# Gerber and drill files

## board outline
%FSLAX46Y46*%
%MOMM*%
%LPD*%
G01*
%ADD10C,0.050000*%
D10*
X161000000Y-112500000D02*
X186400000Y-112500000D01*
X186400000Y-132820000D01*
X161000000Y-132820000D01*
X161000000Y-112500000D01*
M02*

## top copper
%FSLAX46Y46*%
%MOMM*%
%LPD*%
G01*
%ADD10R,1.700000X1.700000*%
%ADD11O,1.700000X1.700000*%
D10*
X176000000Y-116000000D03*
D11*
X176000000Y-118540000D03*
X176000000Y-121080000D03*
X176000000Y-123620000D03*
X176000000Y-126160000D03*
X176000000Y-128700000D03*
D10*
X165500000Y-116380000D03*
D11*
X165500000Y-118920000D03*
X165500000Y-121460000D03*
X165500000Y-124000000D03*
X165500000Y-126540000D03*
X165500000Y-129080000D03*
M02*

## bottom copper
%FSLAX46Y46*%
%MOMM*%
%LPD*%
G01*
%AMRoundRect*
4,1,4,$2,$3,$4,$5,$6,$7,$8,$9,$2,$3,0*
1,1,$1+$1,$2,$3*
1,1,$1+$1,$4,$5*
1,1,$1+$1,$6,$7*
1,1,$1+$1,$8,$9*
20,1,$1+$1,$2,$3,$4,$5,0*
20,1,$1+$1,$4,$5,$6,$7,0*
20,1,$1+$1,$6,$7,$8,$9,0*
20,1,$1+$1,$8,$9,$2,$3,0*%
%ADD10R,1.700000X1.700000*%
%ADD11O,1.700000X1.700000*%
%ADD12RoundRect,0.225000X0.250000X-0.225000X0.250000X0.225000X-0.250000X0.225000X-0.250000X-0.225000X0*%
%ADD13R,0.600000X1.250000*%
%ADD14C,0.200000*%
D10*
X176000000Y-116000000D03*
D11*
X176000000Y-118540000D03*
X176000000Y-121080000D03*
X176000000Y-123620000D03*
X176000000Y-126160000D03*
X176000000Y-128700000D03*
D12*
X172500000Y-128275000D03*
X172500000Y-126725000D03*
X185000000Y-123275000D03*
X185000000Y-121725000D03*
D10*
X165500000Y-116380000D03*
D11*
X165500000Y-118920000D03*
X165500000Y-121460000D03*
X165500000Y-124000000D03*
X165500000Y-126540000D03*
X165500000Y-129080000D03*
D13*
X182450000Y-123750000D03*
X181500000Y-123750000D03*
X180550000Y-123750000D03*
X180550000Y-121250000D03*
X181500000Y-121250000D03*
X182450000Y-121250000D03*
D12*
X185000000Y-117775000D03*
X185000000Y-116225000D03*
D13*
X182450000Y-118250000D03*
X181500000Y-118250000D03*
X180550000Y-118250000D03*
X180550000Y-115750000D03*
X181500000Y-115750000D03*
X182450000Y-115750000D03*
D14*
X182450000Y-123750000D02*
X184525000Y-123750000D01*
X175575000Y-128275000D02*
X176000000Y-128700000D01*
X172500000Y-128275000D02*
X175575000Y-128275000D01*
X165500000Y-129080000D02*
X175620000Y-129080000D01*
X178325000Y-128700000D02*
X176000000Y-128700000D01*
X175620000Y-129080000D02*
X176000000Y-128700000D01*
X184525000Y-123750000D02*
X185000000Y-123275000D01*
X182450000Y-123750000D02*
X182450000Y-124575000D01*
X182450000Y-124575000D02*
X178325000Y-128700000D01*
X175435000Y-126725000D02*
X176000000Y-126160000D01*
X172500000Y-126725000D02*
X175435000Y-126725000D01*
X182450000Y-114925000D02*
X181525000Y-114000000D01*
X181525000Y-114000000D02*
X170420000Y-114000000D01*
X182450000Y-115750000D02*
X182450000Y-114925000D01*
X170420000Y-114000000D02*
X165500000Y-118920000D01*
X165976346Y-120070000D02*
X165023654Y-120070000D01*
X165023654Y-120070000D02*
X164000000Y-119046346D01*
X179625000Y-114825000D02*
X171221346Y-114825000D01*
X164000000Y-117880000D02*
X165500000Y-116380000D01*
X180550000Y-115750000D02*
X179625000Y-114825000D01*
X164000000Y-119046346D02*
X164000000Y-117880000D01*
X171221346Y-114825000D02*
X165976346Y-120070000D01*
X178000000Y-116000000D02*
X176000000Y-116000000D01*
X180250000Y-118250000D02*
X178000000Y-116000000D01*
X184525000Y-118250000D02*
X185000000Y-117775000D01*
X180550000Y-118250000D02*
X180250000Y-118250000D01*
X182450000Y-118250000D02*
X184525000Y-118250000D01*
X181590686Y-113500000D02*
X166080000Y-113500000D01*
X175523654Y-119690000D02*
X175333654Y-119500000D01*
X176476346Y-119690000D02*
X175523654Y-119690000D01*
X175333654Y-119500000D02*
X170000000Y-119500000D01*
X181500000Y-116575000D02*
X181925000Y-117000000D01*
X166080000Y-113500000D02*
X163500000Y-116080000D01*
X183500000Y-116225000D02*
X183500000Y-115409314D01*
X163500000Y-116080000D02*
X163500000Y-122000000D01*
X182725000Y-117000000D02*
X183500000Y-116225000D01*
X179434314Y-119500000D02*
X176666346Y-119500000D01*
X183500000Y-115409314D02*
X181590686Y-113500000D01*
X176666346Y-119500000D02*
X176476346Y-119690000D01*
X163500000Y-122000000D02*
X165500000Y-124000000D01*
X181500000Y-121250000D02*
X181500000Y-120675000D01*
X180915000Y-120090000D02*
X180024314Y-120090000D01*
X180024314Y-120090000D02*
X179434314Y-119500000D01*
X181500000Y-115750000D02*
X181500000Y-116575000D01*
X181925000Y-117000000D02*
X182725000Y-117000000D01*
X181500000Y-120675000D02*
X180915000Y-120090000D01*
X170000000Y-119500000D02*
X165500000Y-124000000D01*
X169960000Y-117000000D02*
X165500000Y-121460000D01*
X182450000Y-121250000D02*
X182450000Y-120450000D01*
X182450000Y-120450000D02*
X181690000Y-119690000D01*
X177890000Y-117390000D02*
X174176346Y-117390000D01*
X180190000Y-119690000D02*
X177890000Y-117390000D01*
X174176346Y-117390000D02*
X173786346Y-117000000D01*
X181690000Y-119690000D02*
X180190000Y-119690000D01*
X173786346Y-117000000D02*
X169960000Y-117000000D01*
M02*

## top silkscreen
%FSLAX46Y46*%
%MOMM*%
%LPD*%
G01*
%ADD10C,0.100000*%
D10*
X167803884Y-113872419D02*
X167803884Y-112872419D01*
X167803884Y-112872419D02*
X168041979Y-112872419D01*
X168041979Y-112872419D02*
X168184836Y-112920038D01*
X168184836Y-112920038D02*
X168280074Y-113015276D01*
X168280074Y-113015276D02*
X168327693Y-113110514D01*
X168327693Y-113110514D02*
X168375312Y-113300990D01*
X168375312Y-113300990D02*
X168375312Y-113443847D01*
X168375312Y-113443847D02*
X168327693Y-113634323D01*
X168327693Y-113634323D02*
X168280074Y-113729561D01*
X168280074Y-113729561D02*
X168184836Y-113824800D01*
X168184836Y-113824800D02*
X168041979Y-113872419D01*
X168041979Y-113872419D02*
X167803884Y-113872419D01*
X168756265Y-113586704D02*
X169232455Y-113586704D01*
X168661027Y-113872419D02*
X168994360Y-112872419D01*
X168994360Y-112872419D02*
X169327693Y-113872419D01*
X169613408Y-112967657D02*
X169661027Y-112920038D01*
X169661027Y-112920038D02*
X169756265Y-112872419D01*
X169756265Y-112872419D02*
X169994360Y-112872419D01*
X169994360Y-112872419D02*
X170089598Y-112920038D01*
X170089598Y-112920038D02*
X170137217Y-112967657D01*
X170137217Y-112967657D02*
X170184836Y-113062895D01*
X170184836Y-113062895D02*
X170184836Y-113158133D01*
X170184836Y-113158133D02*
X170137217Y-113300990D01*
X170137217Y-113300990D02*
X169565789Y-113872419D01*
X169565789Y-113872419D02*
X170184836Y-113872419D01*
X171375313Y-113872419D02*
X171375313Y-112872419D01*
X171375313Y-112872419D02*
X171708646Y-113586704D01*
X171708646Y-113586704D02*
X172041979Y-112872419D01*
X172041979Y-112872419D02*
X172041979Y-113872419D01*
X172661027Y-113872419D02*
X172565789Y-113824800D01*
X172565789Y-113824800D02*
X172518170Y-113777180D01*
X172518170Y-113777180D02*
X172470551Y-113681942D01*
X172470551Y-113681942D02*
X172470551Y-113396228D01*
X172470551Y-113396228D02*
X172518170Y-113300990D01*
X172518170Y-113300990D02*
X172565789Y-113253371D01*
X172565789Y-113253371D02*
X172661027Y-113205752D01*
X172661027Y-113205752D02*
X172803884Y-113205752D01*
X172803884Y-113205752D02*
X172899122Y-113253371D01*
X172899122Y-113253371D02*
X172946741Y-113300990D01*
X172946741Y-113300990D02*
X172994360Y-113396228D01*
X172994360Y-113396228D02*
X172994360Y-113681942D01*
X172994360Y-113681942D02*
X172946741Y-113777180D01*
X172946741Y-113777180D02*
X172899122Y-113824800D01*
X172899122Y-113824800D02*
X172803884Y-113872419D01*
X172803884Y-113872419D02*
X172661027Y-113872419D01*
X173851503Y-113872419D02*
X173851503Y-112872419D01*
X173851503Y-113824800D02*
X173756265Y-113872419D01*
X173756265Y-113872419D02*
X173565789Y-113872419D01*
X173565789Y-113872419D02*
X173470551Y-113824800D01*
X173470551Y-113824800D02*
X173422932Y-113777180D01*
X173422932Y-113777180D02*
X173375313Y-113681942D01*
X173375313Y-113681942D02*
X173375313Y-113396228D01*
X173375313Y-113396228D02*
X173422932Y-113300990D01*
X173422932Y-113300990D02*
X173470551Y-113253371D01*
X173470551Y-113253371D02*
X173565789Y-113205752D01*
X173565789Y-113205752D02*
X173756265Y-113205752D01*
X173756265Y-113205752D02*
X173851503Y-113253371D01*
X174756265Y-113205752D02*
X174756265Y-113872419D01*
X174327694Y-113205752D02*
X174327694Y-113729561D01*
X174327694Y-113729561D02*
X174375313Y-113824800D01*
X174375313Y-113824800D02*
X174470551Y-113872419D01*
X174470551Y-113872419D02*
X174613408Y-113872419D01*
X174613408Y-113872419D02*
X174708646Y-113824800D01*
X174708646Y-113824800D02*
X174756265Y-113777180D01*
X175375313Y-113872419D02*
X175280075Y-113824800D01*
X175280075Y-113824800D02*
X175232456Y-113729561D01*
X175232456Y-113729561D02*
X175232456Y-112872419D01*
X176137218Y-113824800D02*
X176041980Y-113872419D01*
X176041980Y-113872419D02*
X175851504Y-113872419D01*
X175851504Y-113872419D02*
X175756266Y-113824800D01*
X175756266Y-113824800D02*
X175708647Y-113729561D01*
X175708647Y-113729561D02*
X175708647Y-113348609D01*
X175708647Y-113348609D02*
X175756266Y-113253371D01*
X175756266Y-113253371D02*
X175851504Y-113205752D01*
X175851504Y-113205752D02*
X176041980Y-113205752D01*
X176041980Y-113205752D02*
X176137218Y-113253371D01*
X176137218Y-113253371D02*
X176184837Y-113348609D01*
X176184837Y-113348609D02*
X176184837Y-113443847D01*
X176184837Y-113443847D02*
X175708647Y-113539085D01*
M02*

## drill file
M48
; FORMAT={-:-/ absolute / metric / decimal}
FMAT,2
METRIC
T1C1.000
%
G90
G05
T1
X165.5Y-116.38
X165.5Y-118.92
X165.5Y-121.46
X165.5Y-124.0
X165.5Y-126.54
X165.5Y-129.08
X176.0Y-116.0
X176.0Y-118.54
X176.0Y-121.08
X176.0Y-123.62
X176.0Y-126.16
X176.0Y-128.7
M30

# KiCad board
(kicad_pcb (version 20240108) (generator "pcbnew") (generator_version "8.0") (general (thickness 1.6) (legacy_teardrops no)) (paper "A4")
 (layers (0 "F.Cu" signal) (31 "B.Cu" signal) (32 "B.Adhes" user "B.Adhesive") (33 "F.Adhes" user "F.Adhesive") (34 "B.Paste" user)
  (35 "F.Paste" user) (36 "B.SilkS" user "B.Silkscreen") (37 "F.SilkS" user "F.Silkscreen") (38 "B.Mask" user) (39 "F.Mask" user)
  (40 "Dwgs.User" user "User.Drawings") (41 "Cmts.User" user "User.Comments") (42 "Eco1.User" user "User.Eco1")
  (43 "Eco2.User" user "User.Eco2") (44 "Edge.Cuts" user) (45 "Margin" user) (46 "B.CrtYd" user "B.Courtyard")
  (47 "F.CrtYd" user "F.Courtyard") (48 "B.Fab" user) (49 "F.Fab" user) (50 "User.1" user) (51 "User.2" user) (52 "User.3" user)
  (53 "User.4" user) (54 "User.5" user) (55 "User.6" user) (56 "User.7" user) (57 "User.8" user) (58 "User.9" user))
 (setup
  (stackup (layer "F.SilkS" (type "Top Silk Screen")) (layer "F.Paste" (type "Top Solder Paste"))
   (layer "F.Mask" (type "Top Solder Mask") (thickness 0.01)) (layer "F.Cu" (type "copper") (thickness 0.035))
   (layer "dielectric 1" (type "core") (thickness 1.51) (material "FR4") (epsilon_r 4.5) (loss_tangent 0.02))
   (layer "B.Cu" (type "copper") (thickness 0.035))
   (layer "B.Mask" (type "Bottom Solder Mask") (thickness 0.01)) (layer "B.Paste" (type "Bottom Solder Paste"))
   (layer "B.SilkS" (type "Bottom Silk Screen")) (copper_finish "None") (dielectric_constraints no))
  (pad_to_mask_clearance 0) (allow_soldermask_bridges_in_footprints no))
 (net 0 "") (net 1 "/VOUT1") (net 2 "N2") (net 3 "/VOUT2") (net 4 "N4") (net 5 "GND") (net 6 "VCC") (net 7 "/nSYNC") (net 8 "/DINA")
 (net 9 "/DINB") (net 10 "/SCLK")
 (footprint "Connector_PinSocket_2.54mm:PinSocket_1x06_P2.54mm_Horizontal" (layer "B.Cu") (at 176 116 180)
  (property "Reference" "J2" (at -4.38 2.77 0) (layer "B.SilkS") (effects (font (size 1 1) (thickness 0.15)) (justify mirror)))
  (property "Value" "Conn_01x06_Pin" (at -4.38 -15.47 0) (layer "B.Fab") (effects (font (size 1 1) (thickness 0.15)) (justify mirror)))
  (pad "1" thru_hole rect (at 0 0 180) (size 1.7 1.7) (drill 1) (layers "*.Cu" "*.Mask") (remove_unused_layers no) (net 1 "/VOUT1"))
  (pad "2" thru_hole oval (at 0 -2.54 180) (size 1.7 1.7) (drill 1) (layers "*.Cu" "*.Mask") (remove_unused_layers no) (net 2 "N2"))
  (pad "3" thru_hole oval (at 0 -5.08 180) (size 1.7 1.7) (drill 1) (layers "*.Cu" "*.Mask") (remove_unused_layers no) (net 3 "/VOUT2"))
  (pad "4" thru_hole oval (at 0 -7.62 180) (size 1.7 1.7) (drill 1) (layers "*.Cu" "*.Mask") (remove_unused_layers no) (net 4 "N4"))
  (pad "5" thru_hole oval (at 0 -10.16 180) (size 1.7 1.7) (drill 1) (layers "*.Cu" "*.Mask") (remove_unused_layers no) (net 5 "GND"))
  (pad "6" thru_hole oval (at 0 -12.7 180) (size 1.7 1.7) (drill 1) (layers "*.Cu" "*.Mask") (remove_unused_layers no) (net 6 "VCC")))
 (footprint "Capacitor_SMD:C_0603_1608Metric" (layer "B.Cu") (at 172.5 127.5 90)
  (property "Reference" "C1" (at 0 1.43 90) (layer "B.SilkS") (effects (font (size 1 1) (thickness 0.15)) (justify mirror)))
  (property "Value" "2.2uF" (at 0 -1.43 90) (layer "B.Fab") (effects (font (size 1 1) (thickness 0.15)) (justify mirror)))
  (pad "1" smd roundrect (at -0.775 0 90) (size 0.9 0.95) (layers "B.Cu" "B.Paste" "B.Mask") (roundrect_rratio 0.25) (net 6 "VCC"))
  (pad "2" smd roundrect (at 0.775 0 90) (size 0.9 0.95) (layers "B.Cu" "B.Paste" "B.Mask") (roundrect_rratio 0.25) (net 5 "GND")))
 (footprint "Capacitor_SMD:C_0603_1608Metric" (layer "B.Cu") (at 185 122.5 90)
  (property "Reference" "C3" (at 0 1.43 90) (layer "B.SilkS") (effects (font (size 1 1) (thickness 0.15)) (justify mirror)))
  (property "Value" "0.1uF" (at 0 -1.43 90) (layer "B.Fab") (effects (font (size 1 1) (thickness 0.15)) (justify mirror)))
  (pad "1" smd roundrect (at -0.775 0 90) (size 0.9 0.95) (layers "B.Cu" "B.Paste" "B.Mask") (roundrect_rratio 0.25) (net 6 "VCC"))
  (pad "2" smd roundrect (at 0.775 0 90) (size 0.9 0.95) (layers "B.Cu" "B.Paste" "B.Mask") (roundrect_rratio 0.25) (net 5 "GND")))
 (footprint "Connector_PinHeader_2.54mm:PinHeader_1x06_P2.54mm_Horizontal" (layer "B.Cu") (at 165.5 116.38 180)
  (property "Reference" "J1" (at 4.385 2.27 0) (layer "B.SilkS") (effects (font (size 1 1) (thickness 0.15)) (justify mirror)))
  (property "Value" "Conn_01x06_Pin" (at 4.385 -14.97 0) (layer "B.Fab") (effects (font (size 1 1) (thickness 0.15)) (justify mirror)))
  (pad "1" thru_hole rect (at 0 0 180) (size 1.7 1.7) (drill 1) (layers "*.Cu" "*.Mask") (remove_unused_layers no) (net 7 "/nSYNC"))
  (pad "2" thru_hole oval (at 0 -2.54 180) (size 1.7 1.7) (drill 1) (layers "*.Cu" "*.Mask") (remove_unused_layers no) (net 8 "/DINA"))
  (pad "3" thru_hole oval (at 0 -5.08 180) (size 1.7 1.7) (drill 1) (layers "*.Cu" "*.Mask") (remove_unused_layers no) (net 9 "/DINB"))
  (pad "4" thru_hole oval (at 0 -7.62 180) (size 1.7 1.7) (drill 1) (layers "*.Cu" "*.Mask") (remove_unused_layers no) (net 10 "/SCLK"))
  (pad "5" thru_hole oval (at 0 -10.16 180) (size 1.7 1.7) (drill 1) (layers "*.Cu" "*.Mask") (remove_unused_layers no) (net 5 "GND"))
  (pad "6" thru_hole oval (at 0 -12.7 180) (size 1.7 1.7) (drill 1) (layers "*.Cu" "*.Mask") (remove_unused_layers no) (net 6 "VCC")))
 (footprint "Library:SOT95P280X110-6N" (layer "B.Cu") (at 181.5 122.5 90)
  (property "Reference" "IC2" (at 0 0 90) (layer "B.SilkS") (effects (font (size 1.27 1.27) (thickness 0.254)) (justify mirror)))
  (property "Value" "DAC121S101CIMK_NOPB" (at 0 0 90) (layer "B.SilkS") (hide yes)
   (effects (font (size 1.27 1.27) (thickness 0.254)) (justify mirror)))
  (pad "1" smd rect (at -1.25 0.95) (size 0.6 1.25) (layers "B.Cu" "B.Paste" "B.Mask") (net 3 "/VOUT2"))
  (pad "2" smd rect (at -1.25 0) (size 0.6 1.25) (layers "B.Cu" "B.Paste" "B.Mask") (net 5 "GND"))
  (pad "3" smd rect (at -1.25 -0.95) (size 0.6 1.25) (layers "B.Cu" "B.Paste" "B.Mask") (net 6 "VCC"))
  (pad "4" smd rect (at 1.25 -0.95) (size 0.6 1.25) (layers "B.Cu" "B.Paste" "B.Mask") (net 9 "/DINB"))
  (pad "5" smd rect (at 1.25 0) (size 0.6 1.25) (layers "B.Cu" "B.Paste" "B.Mask") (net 10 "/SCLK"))
  (pad "6" smd rect (at 1.25 0.95) (size 0.6 1.25) (layers "B.Cu" "B.Paste" "B.Mask") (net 7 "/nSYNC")))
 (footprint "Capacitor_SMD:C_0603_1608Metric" (layer "B.Cu") (at 185 117 90)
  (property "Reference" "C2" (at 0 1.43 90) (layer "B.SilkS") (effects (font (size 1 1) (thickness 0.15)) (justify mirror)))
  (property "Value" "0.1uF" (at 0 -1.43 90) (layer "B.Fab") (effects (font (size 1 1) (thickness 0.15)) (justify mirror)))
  (pad "1" smd roundrect (at -0.775 0 90) (size 0.9 0.95) (layers "B.Cu" "B.Paste" "B.Mask") (roundrect_rratio 0.25) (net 6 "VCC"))
  (pad "2" smd roundrect (at 0.775 0 90) (size 0.9 0.95) (layers "B.Cu" "B.Paste" "B.Mask") (roundrect_rratio 0.25) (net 5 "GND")))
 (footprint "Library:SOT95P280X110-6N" (layer "B.Cu") (at 181.5 117 90)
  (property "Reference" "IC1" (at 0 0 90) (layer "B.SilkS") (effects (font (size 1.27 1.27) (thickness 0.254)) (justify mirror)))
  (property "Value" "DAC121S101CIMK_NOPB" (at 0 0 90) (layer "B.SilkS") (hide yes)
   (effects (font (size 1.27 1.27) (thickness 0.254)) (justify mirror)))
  (pad "1" smd rect (at -1.25 0.95) (size 0.6 1.25) (layers "B.Cu" "B.Paste" "B.Mask") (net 1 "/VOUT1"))
  (pad "2" smd rect (at -1.25 0) (size 0.6 1.25) (layers "B.Cu" "B.Paste" "B.Mask") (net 5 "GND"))
  (pad "3" smd rect (at -1.25 -0.95) (size 0.6 1.25) (layers "B.Cu" "B.Paste" "B.Mask") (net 6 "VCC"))
  (pad "4" smd rect (at 1.25 -0.95) (size 0.6 1.25) (layers "B.Cu" "B.Paste" "B.Mask") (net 8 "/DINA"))
  (pad "5" smd rect (at 1.25 0) (size 0.6 1.25) (layers "B.Cu" "B.Paste" "B.Mask") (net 10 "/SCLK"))
  (pad "6" smd rect (at 1.25 0.95) (size 0.6 1.25) (layers "B.Cu" "B.Paste" "B.Mask") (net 7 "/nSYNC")))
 (gr_rect (start 161 112.5) (end 186.4 132.82) (stroke (width 0.05) (type default)) (fill none) (layer "Edge.Cuts"))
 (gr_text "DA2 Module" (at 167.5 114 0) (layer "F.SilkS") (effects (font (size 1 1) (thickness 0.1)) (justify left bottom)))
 (segment (start 182.45 123.75) (end 184.525 123.75) (width 0.2) (layer "B.Cu") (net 6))
 (segment (start 175.575 128.275) (end 176 128.7) (width 0.2) (layer "B.Cu") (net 6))
 (segment (start 172.5 128.275) (end 175.575 128.275) (width 0.2) (layer "B.Cu") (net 6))
 (segment (start 165.5 129.08) (end 175.62 129.08) (width 0.2) (layer "B.Cu") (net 6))
 (segment (start 178.325 128.7) (end 176 128.7) (width 0.2) (layer "B.Cu") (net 6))
 (segment (start 175.62 129.08) (end 176 128.7) (width 0.2) (layer "B.Cu") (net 6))
 (segment (start 184.525 123.75) (end 185 123.275) (width 0.2) (layer "B.Cu") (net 6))
 (segment (start 182.45 123.75) (end 182.45 124.575) (width 0.2) (layer "B.Cu") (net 6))
 (segment (start 182.45 124.575) (end 178.325 128.7) (width 0.2) (layer "B.Cu") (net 6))
 (segment (start 175.435 126.725) (end 176 126.16) (width 0.2) (layer "B.Cu") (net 5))
 (segment (start 172.5 126.725) (end 175.435 126.725) (width 0.2) (layer "B.Cu") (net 5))
 (segment (start 182.45 114.925) (end 181.525 114) (width 0.2) (layer "B.Cu") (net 8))
 (segment (start 181.525 114) (end 170.42 114) (width 0.2) (layer "B.Cu") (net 8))
 (segment (start 182.45 115.75) (end 182.45 114.925) (width 0.2) (layer "B.Cu") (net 8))
 (segment (start 170.42 114) (end 165.5 118.92) (width 0.2) (layer "B.Cu") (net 8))
 (segment (start 165.976346 120.07) (end 165.023654 120.07) (width 0.2) (layer "B.Cu") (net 7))
 (segment (start 165.023654 120.07) (end 164 119.046346) (width 0.2) (layer "B.Cu") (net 7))
 (segment (start 179.625 114.825) (end 171.221346 114.825) (width 0.2) (layer "B.Cu") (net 7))
 (segment (start 164 117.88) (end 165.5 116.38) (width 0.2) (layer "B.Cu") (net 7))
 (segment (start 180.55 115.75) (end 179.625 114.825) (width 0.2) (layer "B.Cu") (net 7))
 (segment (start 164 119.046346) (end 164 117.88) (width 0.2) (layer "B.Cu") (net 7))
 (segment (start 171.221346 114.825) (end 165.976346 120.07) (width 0.2) (layer "B.Cu") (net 7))
 (segment (start 178 116) (end 176 116) (width 0.2) (layer "B.Cu") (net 1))
 (segment (start 180.25 118.25) (end 178 116) (width 0.2) (layer "B.Cu") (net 1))
 (segment (start 184.525 118.25) (end 185 117.775) (width 0.2) (layer "B.Cu") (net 1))
 (segment (start 180.55 118.25) (end 180.25 118.25) (width 0.2) (layer "B.Cu") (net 1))
 (segment (start 182.45 118.25) (end 184.525 118.25) (width 0.2) (layer "B.Cu") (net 1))
 (segment (start 181.590686 113.5) (end 166.08 113.5) (width 0.2) (layer "B.Cu") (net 10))
 (segment (start 175.523654 119.69) (end 175.333654 119.5) (width 0.2) (layer "B.Cu") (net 10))
 (segment (start 176.476346 119.69) (end 175.523654 119.69) (width 0.2) (layer "B.Cu") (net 10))
 (segment (start 175.333654 119.5) (end 170 119.5) (width 0.2) (layer "B.Cu") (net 10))
 (segment (start 181.5 116.575) (end 181.925 117) (width 0.2) (layer "B.Cu") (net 10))
 (segment (start 166.08 113.5) (end 163.5 116.08) (width 0.2) (layer "B.Cu") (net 10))
 (segment (start 183.5 116.225) (end 183.5 115.409314) (width 0.2) (layer "B.Cu") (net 10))
 (segment (start 163.5 116.08) (end 163.5 122) (width 0.2) (layer "B.Cu") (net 10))
 (segment (start 182.725 117) (end 183.5 116.225) (width 0.2) (layer "B.Cu") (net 10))
 (segment (start 179.434314 119.5) (end 176.666346 119.5) (width 0.2) (layer "B.Cu") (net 10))
 (segment (start 183.5 115.409314) (end 181.590686 113.5) (width 0.2) (layer "B.Cu") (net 10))
 (segment (start 176.666346 119.5) (end 176.476346 119.69) (width 0.2) (layer "B.Cu") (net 10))
 (segment (start 163.5 122) (end 165.5 124) (width 0.2) (layer "B.Cu") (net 10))
 (segment (start 181.5 121.25) (end 181.5 120.675) (width 0.2) (layer "B.Cu") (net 10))
 (segment (start 180.915 120.09) (end 180.024314 120.09) (width 0.2) (layer "B.Cu") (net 10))
 (segment (start 180.024314 120.09) (end 179.434314 119.5) (width 0.2) (layer "B.Cu") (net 10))
 (segment (start 181.5 115.75) (end 181.5 116.575) (width 0.2) (layer "B.Cu") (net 10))
 (segment (start 181.925 117) (end 182.725 117) (width 0.2) (layer "B.Cu") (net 10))
 (segment (start 181.5 120.675) (end 180.915 120.09) (width 0.2) (layer "B.Cu") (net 10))
 (segment (start 170 119.5) (end 165.5 124) (width 0.2) (layer "B.Cu") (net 10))
 (segment (start 169.96 117) (end 165.5 121.46) (width 0.2) (layer "B.Cu") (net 9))
 (segment (start 182.45 121.25) (end 182.45 120.45) (width 0.2) (layer "B.Cu") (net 9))
 (segment (start 182.45 120.45) (end 181.69 119.69) (width 0.2) (layer "B.Cu") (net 9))
 (segment (start 177.89 117.39) (end 174.176346 117.39) (width 0.2) (layer "B.Cu") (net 9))
 (segment (start 180.19 119.69) (end 177.89 117.39) (width 0.2) (layer "B.Cu") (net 9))
 (segment (start 174.176346 117.39) (end 173.786346 117) (width 0.2) (layer "B.Cu") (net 9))
 (segment (start 181.69 119.69) (end 180.19 119.69) (width 0.2) (layer "B.Cu") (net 9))
 (segment (start 173.786346 117) (end 169.96 117) (width 0.2) (layer "B.Cu") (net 9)))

